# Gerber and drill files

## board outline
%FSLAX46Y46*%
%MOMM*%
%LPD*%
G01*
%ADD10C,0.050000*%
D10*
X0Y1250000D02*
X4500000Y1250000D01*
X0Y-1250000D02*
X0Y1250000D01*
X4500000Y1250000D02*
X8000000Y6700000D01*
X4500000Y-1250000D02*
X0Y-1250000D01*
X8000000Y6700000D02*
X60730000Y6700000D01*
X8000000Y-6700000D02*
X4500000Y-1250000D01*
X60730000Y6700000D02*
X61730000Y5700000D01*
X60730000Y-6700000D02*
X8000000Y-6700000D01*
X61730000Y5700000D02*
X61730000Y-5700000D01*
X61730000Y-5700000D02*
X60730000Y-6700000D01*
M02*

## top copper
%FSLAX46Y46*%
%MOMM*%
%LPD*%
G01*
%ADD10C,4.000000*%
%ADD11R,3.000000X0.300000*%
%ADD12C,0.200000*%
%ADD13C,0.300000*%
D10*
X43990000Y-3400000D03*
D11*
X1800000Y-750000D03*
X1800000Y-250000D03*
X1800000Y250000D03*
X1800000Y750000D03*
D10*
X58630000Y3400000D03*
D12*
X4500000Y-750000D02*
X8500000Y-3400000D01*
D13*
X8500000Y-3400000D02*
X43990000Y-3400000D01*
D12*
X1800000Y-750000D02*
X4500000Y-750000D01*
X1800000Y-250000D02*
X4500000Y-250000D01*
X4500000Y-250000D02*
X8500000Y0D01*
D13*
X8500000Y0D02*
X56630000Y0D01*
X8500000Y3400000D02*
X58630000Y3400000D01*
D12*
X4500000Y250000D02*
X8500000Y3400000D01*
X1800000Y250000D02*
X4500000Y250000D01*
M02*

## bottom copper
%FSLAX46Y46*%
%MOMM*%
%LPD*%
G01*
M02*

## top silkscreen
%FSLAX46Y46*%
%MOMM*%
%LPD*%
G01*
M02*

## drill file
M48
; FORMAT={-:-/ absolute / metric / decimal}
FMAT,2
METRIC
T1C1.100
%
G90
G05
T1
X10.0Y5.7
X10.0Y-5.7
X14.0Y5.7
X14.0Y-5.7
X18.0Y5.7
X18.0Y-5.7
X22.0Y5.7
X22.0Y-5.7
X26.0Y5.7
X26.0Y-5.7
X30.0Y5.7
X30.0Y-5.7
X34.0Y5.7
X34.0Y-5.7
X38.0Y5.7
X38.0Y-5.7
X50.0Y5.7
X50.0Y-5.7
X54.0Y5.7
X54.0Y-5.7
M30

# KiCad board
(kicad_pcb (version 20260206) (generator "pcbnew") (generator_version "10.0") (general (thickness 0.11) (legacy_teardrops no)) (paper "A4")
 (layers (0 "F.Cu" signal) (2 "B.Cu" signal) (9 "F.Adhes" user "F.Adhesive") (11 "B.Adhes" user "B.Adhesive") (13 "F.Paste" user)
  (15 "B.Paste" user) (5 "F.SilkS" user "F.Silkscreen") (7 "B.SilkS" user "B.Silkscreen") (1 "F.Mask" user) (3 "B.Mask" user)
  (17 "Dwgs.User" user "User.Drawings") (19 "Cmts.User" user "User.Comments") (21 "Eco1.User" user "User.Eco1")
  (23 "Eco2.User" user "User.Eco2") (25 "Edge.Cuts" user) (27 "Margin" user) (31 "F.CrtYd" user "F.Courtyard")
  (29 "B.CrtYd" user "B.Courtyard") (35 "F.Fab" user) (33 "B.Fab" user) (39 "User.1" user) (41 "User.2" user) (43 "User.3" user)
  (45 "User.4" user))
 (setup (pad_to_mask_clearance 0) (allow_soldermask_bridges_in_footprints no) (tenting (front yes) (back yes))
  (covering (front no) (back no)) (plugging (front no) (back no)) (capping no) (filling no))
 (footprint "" (layer "F.Cu") (at 22 -5.7)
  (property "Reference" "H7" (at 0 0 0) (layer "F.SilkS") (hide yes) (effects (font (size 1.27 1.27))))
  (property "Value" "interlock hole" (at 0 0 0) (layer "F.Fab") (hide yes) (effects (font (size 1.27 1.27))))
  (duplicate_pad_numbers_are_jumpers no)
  (pad "" np_thru_hole circle (at 0 0) (size 1.1 1.1) (drill 1.1) (layers "*.Cu" "*.Mask")))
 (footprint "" (layer "F.Cu") (at 18 -5.7)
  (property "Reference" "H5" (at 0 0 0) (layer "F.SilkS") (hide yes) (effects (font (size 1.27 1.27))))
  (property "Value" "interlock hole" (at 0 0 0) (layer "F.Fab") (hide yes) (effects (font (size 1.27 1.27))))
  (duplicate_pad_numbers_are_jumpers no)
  (pad "" np_thru_hole circle (at 0 0) (size 1.1 1.1) (drill 1.1) (layers "*.Cu" "*.Mask")))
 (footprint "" (layer "F.Cu") (at 22 5.7)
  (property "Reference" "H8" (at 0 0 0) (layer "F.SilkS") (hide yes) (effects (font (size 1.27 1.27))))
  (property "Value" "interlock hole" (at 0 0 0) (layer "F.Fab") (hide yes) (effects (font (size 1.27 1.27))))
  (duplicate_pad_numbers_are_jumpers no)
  (pad "" np_thru_hole circle (at 0 0) (size 1.1 1.1) (drill 1.1) (layers "*.Cu" "*.Mask")))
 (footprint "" (layer "F.Cu") (at 26 5.7)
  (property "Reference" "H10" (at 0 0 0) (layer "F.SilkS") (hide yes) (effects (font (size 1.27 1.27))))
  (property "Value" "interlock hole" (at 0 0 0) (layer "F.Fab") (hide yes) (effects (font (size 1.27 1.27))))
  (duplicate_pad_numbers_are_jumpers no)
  (pad "" np_thru_hole circle (at 0 0) (size 1.1 1.1) (drill 1.1) (layers "*.Cu" "*.Mask")))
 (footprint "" (layer "F.Cu") (at 43.99 3.4)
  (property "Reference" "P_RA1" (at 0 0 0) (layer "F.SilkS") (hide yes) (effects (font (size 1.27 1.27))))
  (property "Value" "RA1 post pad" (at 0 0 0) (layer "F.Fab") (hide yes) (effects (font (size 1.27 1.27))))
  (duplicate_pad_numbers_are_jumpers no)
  (pad "1" smd circle (at 0 0) (size 4 4) (layers "F.Cu" "F.Mask" "F.Paste") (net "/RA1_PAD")))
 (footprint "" (layer "F.Cu") (at 50 5.7)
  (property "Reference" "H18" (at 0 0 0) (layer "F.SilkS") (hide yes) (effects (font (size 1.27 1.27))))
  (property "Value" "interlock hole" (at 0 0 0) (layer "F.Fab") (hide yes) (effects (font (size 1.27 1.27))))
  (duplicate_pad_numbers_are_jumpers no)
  (pad "" np_thru_hole circle (at 0 0) (size 1.1 1.1) (drill 1.1) (layers "*.Cu" "*.Mask")))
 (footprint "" (layer "F.Cu") (at 10 5.7)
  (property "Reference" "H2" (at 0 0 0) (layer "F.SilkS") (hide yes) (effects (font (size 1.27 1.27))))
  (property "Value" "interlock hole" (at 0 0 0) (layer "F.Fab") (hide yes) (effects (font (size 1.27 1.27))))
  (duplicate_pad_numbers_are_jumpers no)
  (pad "" np_thru_hole circle (at 0 0) (size 1.1 1.1) (drill 1.1) (layers "*.Cu" "*.Mask")))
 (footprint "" (layer "F.Cu") (at 38 -5.7)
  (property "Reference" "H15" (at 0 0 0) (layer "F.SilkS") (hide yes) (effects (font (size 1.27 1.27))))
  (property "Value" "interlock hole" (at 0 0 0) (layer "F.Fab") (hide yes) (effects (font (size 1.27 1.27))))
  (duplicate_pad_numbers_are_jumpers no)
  (pad "" np_thru_hole circle (at 0 0) (size 1.1 1.1) (drill 1.1) (layers "*.Cu" "*.Mask")))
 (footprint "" (layer "F.Cu") (at 54 5.7)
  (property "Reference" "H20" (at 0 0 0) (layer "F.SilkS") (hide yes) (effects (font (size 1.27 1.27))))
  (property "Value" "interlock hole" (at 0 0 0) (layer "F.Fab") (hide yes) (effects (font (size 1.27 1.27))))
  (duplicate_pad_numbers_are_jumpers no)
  (pad "" np_thru_hole circle (at 0 0) (size 1.1 1.1) (drill 1.1) (layers "*.Cu" "*.Mask")))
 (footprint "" (layer "F.Cu") (at 14 5.7)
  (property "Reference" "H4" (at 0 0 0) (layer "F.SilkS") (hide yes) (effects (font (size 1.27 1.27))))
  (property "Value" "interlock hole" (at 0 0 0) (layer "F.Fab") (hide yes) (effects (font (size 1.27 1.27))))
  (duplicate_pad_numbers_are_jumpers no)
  (pad "" np_thru_hole circle (at 0 0) (size 1.1 1.1) (drill 1.1) (layers "*.Cu" "*.Mask")))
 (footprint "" (layer "F.Cu") (at 26 -5.7)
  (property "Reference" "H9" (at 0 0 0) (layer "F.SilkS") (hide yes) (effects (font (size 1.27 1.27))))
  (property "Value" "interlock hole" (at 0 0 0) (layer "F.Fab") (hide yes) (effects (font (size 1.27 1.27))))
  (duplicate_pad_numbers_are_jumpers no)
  (pad "" np_thru_hole circle (at 0 0) (size 1.1 1.1) (drill 1.1) (layers "*.Cu" "*.Mask")))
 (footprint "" (layer "F.Cu") (at 30 -5.7)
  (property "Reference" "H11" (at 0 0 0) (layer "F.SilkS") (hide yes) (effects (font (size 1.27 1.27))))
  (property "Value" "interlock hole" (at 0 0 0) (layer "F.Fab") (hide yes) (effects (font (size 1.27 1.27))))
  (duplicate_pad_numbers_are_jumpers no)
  (pad "" np_thru_hole circle (at 0 0) (size 1.1 1.1) (drill 1.1) (layers "*.Cu" "*.Mask")))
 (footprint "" (layer "F.Cu") (at 34 5.7)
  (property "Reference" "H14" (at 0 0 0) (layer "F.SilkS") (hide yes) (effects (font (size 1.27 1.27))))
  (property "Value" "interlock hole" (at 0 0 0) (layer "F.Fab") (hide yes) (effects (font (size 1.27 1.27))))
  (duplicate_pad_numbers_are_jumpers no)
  (pad "" np_thru_hole circle (at 0 0) (size 1.1 1.1) (drill 1.1) (layers "*.Cu" "*.Mask")))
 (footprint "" (layer "F.Cu") (at 30 5.7)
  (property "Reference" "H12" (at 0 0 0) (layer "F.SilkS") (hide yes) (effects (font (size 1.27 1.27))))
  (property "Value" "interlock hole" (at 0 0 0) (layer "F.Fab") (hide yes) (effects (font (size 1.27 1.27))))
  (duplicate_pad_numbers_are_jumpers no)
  (pad "" np_thru_hole circle (at 0 0) (size 1.1 1.1) (drill 1.1) (layers "*.Cu" "*.Mask")))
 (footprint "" (layer "F.Cu") (at 50 -5.7)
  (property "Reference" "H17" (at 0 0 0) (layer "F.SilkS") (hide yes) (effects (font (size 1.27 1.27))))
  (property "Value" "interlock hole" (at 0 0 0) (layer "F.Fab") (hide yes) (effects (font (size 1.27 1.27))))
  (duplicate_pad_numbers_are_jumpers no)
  (pad "" np_thru_hole circle (at 0 0) (size 1.1 1.1) (drill 1.1) (layers "*.Cu" "*.Mask")))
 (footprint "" (layer "F.Cu") (at 34 -5.7)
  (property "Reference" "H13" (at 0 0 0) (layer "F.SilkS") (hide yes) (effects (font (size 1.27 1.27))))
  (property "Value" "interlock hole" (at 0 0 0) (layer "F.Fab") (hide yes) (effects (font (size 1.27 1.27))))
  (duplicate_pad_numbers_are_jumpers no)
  (pad "" np_thru_hole circle (at 0 0) (size 1.1 1.1) (drill 1.1) (layers "*.Cu" "*.Mask")))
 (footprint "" (layer "F.Cu") (at 18 5.7)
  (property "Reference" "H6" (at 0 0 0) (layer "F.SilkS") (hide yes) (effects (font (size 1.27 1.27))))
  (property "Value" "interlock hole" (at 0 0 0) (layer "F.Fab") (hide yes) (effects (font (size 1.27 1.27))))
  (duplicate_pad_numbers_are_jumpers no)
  (pad "" np_thru_hole circle (at 0 0) (size 1.1 1.1) (drill 1.1) (layers "*.Cu" "*.Mask")))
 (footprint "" (layer "F.Cu") (at 54 -5.7)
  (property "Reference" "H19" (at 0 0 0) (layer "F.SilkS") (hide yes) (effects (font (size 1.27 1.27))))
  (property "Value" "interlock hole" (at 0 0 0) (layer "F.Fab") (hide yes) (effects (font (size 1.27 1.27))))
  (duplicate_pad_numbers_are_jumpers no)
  (pad "" np_thru_hole circle (at 0 0) (size 1.1 1.1) (drill 1.1) (layers "*.Cu" "*.Mask")))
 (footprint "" (layer "F.Cu") (at 10 -5.7)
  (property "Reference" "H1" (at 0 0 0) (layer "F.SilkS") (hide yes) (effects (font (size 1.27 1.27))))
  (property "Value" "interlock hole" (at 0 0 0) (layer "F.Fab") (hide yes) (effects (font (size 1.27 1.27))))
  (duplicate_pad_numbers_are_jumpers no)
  (pad "" np_thru_hole circle (at 0 0) (size 1.1 1.1) (drill 1.1) (layers "*.Cu" "*.Mask")))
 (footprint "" (layer "F.Cu") (at 14 -5.7)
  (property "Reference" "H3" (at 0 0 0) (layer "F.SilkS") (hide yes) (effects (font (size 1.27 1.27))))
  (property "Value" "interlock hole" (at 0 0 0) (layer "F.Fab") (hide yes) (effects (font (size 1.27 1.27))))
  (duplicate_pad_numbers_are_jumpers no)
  (pad "" np_thru_hole circle (at 0 0) (size 1.1 1.1) (drill 1.1) (layers "*.Cu" "*.Mask")))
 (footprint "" (layer "F.Cu") (at 1.8 0)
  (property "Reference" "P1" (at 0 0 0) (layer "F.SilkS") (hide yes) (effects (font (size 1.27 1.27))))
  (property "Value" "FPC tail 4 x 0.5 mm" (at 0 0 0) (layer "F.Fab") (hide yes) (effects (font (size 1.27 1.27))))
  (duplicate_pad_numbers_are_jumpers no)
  (pad "1" smd rect (at 0 0.75) (size 3 0.3) (layers "F.Cu" "F.Mask" "F.Paste") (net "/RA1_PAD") (thermal_bridge_angle 45))
  (pad "2" smd rect (at 0 0.25) (size 3 0.3) (layers "F.Cu" "F.Mask" "F.Paste") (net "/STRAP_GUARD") (thermal_bridge_angle 45))
  (pad "3" smd rect (at 0 -0.25) (size 3 0.3) (layers "F.Cu" "F.Mask" "F.Paste") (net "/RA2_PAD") (thermal_bridge_angle 45))
  (pad "4" smd rect (at 0 -0.75) (size 3 0.3) (layers "F.Cu" "F.Mask" "F.Paste") (thermal_bridge_angle 45)))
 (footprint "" (layer "F.Cu") (at 38 5.7)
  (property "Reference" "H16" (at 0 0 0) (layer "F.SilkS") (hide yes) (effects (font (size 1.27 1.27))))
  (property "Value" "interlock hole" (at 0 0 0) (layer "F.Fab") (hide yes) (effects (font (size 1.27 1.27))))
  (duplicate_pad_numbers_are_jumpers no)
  (pad "" np_thru_hole circle (at 0 0) (size 1.1 1.1) (drill 1.1) (layers "*.Cu" "*.Mask")))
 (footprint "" (layer "F.Cu") (at 58.63 -3.4)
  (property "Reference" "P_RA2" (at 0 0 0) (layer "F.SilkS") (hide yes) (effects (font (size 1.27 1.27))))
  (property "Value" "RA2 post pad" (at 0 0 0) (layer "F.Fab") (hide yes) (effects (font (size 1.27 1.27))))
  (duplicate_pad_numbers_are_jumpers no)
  (pad "1" smd circle (at 0 0) (size 4 4) (layers "F.Cu" "F.Mask" "F.Paste") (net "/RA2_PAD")))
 (gr_line (start 0 -1.25) (end 4.5 -1.25) (stroke (width 0.05) (type default)) (layer "Edge.Cuts"))
 (gr_line (start 0 1.25) (end 0 -1.25) (stroke (width 0.05) (type default)) (layer "Edge.Cuts"))
 (gr_line (start 4.5 -1.25) (end 8 -6.7) (stroke (width 0.05) (type default)) (layer "Edge.Cuts"))
 (gr_line (start 4.5 1.25) (end 0 1.25) (stroke (width 0.05) (type default)) (layer "Edge.Cuts"))
 (gr_line (start 8 -6.7) (end 60.73 -6.7) (stroke (width 0.05) (type default)) (layer "Edge.Cuts"))
 (gr_line (start 8 6.7) (end 4.5 1.25) (stroke (width 0.05) (type default)) (layer "Edge.Cuts"))
 (gr_line (start 60.73 -6.7) (end 61.73 -5.7) (stroke (width 0.05) (type default)) (layer "Edge.Cuts"))
 (gr_line (start 60.73 6.7) (end 8 6.7) (stroke (width 0.05) (type default)) (layer "Edge.Cuts"))
 (gr_line (start 61.73 -5.7) (end 61.73 5.7) (stroke (width 0.05) (type default)) (layer "Edge.Cuts"))
 (gr_line (start 61.73 5.7) (end 60.73 6.7) (stroke (width 0.05) (type default)) (layer "Edge.Cuts"))
 (segment (start 4.5 0.75) (end 8.5 3.4) (width 0.2) (layer "F.Cu") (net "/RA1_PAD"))
 (segment (start 8.5 3.4) (end 43.99 3.4) (width 0.3) (layer "F.Cu") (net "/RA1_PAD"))
 (segment (start 1.8 0.75) (end 4.5 0.75) (width 0.2) (layer "F.Cu") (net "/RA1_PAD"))
 (segment (start 1.8 0.25) (end 4.5 0.25) (width 0.2) (layer "F.Cu") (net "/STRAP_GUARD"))
 (segment (start 4.5 0.25) (end 8.5 0) (width 0.2) (layer "F.Cu") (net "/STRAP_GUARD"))
 (segment (start 8.5 0) (end 56.63 0) (width 0.3) (layer "F.Cu") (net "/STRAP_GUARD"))
 (segment (start 8.5 -3.4) (end 58.63 -3.4) (width 0.3) (layer "F.Cu") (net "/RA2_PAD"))
 (segment (start 4.5 -0.25) (end 8.5 -3.4) (width 0.2) (layer "F.Cu") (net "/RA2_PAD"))
 (segment (start 1.8 -0.25) (end 4.5 -0.25) (width 0.2) (layer "F.Cu") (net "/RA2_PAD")))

